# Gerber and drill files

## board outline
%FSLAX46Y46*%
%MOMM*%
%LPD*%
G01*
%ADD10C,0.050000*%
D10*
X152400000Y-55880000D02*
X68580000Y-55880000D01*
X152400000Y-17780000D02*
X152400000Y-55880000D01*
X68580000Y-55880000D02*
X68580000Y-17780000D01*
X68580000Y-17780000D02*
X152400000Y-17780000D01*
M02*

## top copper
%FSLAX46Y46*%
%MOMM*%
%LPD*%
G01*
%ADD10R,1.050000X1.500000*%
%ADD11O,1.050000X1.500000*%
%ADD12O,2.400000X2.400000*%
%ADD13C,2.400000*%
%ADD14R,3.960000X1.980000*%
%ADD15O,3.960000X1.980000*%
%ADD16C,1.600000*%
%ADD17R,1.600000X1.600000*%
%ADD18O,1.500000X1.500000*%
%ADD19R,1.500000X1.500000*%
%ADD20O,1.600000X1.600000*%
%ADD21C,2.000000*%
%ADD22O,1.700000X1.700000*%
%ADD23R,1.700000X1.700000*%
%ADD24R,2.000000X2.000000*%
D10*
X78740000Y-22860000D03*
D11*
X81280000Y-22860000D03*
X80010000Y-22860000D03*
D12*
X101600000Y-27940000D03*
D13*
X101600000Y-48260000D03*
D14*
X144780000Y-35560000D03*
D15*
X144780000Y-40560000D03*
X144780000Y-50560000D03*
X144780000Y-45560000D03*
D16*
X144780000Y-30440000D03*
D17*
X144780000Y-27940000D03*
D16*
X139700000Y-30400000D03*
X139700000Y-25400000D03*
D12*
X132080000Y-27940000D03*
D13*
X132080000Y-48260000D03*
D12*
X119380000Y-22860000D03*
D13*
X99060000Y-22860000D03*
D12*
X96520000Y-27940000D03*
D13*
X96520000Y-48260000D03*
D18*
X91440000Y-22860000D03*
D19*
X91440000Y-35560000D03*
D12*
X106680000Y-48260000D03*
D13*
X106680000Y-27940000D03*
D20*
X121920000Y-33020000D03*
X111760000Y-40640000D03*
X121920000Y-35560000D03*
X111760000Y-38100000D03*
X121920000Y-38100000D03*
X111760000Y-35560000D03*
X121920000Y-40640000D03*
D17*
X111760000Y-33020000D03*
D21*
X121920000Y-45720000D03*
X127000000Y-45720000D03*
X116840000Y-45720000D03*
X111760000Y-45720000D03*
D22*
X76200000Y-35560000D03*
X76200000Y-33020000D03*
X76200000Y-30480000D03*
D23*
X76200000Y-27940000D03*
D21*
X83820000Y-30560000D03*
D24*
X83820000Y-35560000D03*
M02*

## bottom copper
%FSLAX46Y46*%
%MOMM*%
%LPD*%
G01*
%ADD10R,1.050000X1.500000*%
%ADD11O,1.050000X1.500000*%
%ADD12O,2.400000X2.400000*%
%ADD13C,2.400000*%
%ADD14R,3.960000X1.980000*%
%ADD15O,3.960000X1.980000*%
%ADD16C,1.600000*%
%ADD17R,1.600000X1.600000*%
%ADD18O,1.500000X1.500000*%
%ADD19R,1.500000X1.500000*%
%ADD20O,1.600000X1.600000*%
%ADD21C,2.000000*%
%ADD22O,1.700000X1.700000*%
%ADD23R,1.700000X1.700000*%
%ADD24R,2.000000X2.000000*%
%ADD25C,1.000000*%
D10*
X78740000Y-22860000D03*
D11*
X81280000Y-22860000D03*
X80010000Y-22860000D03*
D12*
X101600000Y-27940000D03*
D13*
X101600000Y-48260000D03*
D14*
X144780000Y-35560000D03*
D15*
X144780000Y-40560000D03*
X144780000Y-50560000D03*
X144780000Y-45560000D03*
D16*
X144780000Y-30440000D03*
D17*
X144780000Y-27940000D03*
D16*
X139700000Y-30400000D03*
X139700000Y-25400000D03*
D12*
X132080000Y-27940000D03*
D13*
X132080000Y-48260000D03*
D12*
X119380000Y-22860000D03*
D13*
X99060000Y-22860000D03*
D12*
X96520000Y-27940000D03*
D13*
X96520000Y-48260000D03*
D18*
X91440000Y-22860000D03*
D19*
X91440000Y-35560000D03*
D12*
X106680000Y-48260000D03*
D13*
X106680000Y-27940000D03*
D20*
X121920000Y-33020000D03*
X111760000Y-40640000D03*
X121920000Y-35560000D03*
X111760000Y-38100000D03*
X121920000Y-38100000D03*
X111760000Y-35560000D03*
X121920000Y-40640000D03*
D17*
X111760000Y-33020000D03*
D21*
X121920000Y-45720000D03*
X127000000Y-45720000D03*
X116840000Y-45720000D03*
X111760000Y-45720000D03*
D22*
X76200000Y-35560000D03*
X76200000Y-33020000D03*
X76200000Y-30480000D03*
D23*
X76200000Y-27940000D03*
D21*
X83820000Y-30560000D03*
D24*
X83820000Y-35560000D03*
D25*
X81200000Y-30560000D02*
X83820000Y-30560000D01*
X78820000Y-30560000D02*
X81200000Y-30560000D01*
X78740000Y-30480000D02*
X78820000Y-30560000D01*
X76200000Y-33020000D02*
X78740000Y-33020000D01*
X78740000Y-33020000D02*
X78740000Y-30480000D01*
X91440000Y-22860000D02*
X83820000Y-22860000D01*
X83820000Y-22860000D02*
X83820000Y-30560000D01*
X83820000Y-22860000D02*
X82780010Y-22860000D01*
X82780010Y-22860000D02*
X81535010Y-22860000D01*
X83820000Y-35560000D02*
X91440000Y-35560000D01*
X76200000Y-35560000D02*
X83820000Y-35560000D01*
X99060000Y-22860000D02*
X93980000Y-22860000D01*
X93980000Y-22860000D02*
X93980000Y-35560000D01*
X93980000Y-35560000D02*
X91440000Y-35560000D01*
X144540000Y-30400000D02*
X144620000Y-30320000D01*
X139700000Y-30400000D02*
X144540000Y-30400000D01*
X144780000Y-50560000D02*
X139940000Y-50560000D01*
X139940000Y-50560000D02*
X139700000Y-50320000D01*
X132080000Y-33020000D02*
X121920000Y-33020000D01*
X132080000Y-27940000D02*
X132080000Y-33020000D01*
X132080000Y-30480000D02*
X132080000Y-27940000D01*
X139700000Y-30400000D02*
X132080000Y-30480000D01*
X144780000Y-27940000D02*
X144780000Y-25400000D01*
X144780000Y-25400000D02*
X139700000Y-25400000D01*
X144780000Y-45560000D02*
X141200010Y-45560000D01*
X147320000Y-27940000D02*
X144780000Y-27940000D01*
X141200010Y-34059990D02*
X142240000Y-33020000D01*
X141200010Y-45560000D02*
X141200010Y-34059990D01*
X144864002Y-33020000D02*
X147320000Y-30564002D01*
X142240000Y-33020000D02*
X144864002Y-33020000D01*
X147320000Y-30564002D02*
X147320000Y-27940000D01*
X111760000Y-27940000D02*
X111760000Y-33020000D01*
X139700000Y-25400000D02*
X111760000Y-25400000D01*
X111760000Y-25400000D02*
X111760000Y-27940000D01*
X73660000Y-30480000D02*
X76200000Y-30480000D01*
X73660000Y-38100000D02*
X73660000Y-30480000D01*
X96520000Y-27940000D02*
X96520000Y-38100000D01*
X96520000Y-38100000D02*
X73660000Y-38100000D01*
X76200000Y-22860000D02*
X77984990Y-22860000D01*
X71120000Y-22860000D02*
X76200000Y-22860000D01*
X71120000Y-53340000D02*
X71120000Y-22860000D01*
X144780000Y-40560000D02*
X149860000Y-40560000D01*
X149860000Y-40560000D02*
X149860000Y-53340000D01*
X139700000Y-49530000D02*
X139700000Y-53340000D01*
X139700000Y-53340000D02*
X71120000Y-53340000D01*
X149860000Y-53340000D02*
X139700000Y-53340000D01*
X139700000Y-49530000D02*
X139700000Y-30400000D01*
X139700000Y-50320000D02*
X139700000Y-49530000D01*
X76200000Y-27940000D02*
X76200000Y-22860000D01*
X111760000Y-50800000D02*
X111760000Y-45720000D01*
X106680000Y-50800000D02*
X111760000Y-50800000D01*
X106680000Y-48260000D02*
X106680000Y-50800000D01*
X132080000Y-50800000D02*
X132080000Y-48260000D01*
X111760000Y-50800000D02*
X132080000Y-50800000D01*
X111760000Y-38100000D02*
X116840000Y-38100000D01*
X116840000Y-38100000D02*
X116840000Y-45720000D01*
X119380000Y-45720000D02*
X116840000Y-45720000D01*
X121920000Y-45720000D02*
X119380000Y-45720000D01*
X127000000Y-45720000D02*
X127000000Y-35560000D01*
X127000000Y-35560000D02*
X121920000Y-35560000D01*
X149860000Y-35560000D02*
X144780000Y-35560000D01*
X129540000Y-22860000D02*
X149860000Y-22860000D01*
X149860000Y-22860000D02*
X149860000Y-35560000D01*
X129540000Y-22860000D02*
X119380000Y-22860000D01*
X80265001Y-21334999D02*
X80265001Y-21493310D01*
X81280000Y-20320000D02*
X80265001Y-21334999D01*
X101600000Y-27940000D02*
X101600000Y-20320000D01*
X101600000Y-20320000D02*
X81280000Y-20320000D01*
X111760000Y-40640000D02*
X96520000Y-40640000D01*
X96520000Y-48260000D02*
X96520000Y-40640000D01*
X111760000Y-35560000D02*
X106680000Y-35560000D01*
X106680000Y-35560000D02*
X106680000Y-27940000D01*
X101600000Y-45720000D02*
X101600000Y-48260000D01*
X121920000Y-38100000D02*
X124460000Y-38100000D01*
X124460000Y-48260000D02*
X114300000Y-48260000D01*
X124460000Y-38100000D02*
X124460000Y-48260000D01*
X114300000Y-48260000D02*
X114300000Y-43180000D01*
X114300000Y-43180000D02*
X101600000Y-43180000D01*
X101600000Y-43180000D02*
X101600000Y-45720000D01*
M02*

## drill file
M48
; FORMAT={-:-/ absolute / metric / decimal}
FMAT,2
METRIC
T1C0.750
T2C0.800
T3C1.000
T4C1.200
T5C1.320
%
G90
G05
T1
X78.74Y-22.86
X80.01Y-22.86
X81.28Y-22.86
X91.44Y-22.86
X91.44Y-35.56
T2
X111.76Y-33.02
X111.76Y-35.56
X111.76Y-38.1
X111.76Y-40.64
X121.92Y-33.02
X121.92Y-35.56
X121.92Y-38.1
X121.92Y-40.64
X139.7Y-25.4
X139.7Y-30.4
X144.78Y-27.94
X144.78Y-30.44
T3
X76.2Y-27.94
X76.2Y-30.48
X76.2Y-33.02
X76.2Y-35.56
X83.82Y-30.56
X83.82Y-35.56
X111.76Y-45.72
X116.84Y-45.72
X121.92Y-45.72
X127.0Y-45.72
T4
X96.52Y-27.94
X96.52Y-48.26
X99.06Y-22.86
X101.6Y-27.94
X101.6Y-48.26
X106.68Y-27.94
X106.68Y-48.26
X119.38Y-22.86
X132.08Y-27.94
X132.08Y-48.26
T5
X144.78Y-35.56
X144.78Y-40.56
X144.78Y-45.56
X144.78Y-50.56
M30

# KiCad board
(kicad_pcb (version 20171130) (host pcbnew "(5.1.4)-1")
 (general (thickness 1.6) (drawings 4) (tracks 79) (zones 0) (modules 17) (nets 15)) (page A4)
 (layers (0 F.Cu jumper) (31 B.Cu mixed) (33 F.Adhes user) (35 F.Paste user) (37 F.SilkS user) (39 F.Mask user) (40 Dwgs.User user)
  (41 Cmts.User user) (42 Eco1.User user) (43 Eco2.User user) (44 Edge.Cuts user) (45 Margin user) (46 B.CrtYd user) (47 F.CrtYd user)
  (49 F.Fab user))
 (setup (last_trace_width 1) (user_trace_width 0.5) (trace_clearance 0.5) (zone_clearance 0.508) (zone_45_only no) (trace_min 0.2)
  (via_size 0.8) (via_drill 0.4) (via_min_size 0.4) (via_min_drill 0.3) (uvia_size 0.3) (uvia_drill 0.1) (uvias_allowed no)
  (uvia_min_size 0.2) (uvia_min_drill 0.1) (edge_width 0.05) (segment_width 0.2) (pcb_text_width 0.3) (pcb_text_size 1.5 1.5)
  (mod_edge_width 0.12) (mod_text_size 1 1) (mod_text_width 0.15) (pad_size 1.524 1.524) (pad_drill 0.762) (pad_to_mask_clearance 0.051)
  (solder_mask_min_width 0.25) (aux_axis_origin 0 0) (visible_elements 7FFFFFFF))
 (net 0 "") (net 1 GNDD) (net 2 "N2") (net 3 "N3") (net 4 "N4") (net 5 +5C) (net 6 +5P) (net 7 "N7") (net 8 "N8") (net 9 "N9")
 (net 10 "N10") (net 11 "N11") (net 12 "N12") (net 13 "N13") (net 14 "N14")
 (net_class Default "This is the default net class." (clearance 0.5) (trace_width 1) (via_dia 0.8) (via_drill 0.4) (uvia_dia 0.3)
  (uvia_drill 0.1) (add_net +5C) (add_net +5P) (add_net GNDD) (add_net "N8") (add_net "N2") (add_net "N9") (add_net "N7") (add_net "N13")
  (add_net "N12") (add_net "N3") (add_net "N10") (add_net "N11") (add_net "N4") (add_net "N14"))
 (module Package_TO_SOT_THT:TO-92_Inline (layer F.Cu) (at 78.74 22.86)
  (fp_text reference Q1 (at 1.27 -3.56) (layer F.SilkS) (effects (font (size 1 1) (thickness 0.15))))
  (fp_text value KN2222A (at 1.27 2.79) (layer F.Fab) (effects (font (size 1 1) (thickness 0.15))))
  (pad 1 thru_hole rect (at 0 0) (size 1.05 1.5) (drill 0.75) (layers *.Cu *.Mask) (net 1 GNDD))
  (pad 3 thru_hole oval (at 2.54 0) (size 1.05 1.5) (drill 0.75) (layers *.Cu *.Mask) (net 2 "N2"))
  (pad 2 thru_hole oval (at 1.27 0) (size 1.05 1.5) (drill 0.75) (layers *.Cu *.Mask) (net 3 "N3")))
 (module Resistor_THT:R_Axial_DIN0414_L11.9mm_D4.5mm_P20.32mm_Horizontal (layer F.Cu) (at 101.6 48.26 90)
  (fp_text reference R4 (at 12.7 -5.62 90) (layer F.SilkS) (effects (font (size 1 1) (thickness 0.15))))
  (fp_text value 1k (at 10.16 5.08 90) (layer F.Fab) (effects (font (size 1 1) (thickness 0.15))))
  (pad 2 thru_hole oval (at 20.32 0 90) (size 2.4 2.4) (drill 1.2) (layers *.Cu *.Mask) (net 3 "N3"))
  (pad 1 thru_hole circle (at 0 0 90) (size 2.4 2.4) (drill 1.2) (layers *.Cu *.Mask) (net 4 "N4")))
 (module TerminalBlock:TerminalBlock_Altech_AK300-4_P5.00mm (layer F.Cu) (at 144.78 35.56 270)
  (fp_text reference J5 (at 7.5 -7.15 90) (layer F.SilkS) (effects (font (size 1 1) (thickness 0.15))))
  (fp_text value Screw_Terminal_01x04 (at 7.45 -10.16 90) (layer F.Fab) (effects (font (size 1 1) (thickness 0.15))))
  (pad 1 thru_hole rect (at 0 0 270) (size 1.98 3.96) (drill 1.32) (layers *.Cu *.Mask) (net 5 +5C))
  (pad 2 thru_hole oval (at 5 0 270) (size 1.98 3.96) (drill 1.32) (layers *.Cu *.Mask) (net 1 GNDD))
  (pad 4 thru_hole oval (at 15 0 270) (size 1.98 3.96) (drill 1.32) (layers *.Cu *.Mask) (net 1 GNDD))
  (pad 3 thru_hole oval (at 10 0 270) (size 1.98 3.96) (drill 1.32) (layers *.Cu *.Mask) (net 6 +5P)))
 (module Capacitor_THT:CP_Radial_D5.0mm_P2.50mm (layer F.Cu) (at 144.78 27.94 270)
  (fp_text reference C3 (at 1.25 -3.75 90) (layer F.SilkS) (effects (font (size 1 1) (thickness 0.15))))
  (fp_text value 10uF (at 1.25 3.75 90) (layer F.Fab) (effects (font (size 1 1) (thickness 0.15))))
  (pad 2 thru_hole circle (at 2.5 0 270) (size 1.6 1.6) (drill 0.8) (layers *.Cu *.Mask) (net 1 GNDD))
  (pad 1 thru_hole rect (at 0 0 270) (size 1.6 1.6) (drill 0.8) (layers *.Cu *.Mask) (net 6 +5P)))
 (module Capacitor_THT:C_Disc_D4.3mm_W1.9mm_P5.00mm (layer F.Cu) (at 139.7 25.4 270)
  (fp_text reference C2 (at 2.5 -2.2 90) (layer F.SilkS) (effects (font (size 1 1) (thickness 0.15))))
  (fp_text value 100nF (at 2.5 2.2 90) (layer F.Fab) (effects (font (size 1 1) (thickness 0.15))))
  (pad 2 thru_hole circle (at 5 0 270) (size 1.6 1.6) (drill 0.8) (layers *.Cu *.Mask) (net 1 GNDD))
  (pad 1 thru_hole circle (at 0 0 270) (size 1.6 1.6) (drill 0.8) (layers *.Cu *.Mask) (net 6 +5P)))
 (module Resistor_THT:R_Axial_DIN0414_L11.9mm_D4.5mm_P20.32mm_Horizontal (layer F.Cu) (at 132.08 48.26 90)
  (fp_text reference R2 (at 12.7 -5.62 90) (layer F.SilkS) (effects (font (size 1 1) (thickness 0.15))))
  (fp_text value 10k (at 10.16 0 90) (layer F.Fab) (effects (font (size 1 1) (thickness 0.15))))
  (pad 2 thru_hole oval (at 20.32 0 90) (size 2.4 2.4) (drill 1.2) (layers *.Cu *.Mask) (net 1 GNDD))
  (pad 1 thru_hole circle (at 0 0 90) (size 2.4 2.4) (drill 1.2) (layers *.Cu *.Mask) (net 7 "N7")))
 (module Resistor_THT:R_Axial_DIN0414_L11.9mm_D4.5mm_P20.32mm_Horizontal (layer F.Cu) (at 99.06 22.86)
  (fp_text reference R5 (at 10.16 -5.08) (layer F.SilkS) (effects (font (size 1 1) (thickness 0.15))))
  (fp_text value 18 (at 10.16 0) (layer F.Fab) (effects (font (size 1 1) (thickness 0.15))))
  (pad 2 thru_hole oval (at 20.32 0) (size 2.4 2.4) (drill 1.2) (layers *.Cu *.Mask) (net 5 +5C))
  (pad 1 thru_hole circle (at 0 0) (size 2.4 2.4) (drill 1.2) (layers *.Cu *.Mask) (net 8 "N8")))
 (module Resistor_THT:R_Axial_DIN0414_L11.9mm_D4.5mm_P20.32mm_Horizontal (layer F.Cu) (at 96.52 48.26 90)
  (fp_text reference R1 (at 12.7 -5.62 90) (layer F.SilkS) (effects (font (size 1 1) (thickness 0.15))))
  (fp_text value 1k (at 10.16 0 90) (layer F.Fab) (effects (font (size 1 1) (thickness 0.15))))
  (pad 2 thru_hole oval (at 20.32 0 90) (size 2.4 2.4) (drill 1.2) (layers *.Cu *.Mask) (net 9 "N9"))
  (pad 1 thru_hole circle (at 0 0 90) (size 2.4 2.4) (drill 1.2) (layers *.Cu *.Mask) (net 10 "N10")))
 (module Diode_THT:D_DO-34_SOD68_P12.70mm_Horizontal (layer F.Cu) (at 91.44 35.56 90)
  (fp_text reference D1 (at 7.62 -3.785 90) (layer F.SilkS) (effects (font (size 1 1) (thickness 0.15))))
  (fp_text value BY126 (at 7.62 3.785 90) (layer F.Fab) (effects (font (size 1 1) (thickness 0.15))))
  (pad 2 thru_hole oval (at 12.7 0 90) (size 1.5 1.5) (drill 0.75) (layers *.Cu *.Mask) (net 2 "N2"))
  (pad 1 thru_hole rect (at 0 0 90) (size 1.5 1.5) (drill 0.75) (layers *.Cu *.Mask) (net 8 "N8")))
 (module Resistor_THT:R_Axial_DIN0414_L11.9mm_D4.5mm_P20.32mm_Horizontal (layer F.Cu) (at 106.68 27.94 270)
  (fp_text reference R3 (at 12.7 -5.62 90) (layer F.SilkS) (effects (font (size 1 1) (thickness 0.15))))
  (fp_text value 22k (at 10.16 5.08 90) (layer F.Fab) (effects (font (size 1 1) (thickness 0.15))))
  (pad 2 thru_hole oval (at 20.32 0 270) (size 2.4 2.4) (drill 1.2) (layers *.Cu *.Mask) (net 7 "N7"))
  (pad 1 thru_hole circle (at 0 0 270) (size 2.4 2.4) (drill 1.2) (layers *.Cu *.Mask) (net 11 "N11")))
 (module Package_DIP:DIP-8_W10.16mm (layer F.Cu) (at 111.76 33.02)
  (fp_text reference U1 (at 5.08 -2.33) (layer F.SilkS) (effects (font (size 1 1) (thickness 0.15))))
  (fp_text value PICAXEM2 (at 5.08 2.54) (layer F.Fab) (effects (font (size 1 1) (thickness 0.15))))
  (pad 8 thru_hole oval (at 10.16 0) (size 1.6 1.6) (drill 0.8) (layers *.Cu *.Mask) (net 1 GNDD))
  (pad 4 thru_hole oval (at 0 7.62) (size 1.6 1.6) (drill 0.8) (layers *.Cu *.Mask) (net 10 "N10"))
  (pad 7 thru_hole oval (at 10.16 2.54) (size 1.6 1.6) (drill 0.8) (layers *.Cu *.Mask) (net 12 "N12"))
  (pad 3 thru_hole oval (at 0 5.08) (size 1.6 1.6) (drill 0.8) (layers *.Cu *.Mask) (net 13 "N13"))
  (pad 6 thru_hole oval (at 10.16 5.08) (size 1.6 1.6) (drill 0.8) (layers *.Cu *.Mask) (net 4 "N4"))
  (pad 2 thru_hole oval (at 0 2.54) (size 1.6 1.6) (drill 0.8) (layers *.Cu *.Mask) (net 11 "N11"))
  (pad 5 thru_hole oval (at 10.16 7.62) (size 1.6 1.6) (drill 0.8) (layers *.Cu *.Mask) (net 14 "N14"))
  (pad 1 thru_hole rect (at 0 0) (size 1.6 1.6) (drill 0.8) (layers *.Cu *.Mask) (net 6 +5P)))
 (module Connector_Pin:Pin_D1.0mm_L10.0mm (layer F.Cu) (at 121.92 45.72)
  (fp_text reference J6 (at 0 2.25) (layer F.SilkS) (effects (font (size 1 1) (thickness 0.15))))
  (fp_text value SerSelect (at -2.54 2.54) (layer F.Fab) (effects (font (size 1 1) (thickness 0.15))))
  (pad 1 thru_hole circle (at 0 0) (size 2 2) (drill 1) (layers *.Cu *.Mask) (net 13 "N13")))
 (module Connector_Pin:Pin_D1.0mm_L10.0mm (layer F.Cu) (at 127 45.72)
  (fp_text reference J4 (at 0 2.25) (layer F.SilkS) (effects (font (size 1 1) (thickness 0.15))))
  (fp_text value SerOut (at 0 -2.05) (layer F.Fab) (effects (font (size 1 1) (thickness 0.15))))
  (pad 1 thru_hole circle (at 0 0) (size 2 2) (drill 1) (layers *.Cu *.Mask) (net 12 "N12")))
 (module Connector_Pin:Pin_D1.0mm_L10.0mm (layer F.Cu) (at 116.84 45.72)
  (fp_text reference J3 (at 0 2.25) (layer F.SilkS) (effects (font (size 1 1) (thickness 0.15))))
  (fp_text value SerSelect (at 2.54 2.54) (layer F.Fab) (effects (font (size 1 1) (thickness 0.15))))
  (pad 1 thru_hole circle (at 0 0) (size 2 2) (drill 1) (layers *.Cu *.Mask) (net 13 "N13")))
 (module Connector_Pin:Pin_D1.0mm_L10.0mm (layer F.Cu) (at 111.76 45.72)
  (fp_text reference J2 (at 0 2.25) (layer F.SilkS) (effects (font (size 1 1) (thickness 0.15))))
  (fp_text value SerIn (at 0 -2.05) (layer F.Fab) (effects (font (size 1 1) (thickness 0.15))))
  (pad 1 thru_hole circle (at 0 0) (size 2 2) (drill 1) (layers *.Cu *.Mask) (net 7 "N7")))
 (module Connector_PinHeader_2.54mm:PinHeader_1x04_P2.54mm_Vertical (layer F.Cu) (at 76.2 27.94)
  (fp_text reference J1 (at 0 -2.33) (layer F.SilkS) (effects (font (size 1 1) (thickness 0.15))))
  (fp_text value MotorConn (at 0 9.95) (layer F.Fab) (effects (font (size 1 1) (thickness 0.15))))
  (pad 4 thru_hole oval (at 0 7.62) (size 1.7 1.7) (drill 1) (layers *.Cu *.Mask) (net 8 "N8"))
  (pad 3 thru_hole oval (at 0 5.08) (size 1.7 1.7) (drill 1) (layers *.Cu *.Mask) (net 2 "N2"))
  (pad 2 thru_hole oval (at 0 2.54) (size 1.7 1.7) (drill 1) (layers *.Cu *.Mask) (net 9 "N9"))
  (pad 1 thru_hole rect (at 0 0) (size 1.7 1.7) (drill 1) (layers *.Cu *.Mask) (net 1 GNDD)))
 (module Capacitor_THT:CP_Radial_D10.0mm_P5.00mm (layer F.Cu) (at 83.82 35.56 90)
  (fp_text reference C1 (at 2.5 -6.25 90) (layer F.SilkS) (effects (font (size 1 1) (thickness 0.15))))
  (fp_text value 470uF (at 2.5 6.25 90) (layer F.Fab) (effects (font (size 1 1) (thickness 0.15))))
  (pad 2 thru_hole circle (at 5 0 90) (size 2 2) (drill 1) (layers *.Cu *.Mask) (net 2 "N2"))
  (pad 1 thru_hole rect (at 0 0 90) (size 2 2) (drill 1) (layers *.Cu *.Mask) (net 8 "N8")))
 (gr_line (start 152.4 55.88) (end 68.58 55.88) (layer Edge.Cuts) (width 0.05))
 (gr_line (start 152.4 17.78) (end 152.4 55.88) (layer Edge.Cuts) (width 0.05))
 (gr_line (start 68.58 55.88) (end 68.58 17.78) (layer Edge.Cuts) (width 0.05))
 (gr_line (start 68.58 17.78) (end 152.4 17.78) (layer Edge.Cuts) (width 0.05))
 (segment (start 81.2 30.56) (end 83.82 30.56) (width 1) (layer B.Cu) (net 2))
 (segment (start 78.82 30.56) (end 81.2 30.56) (width 1) (layer B.Cu) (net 2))
 (segment (start 78.74 30.48) (end 78.82 30.56) (width 1) (layer B.Cu) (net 2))
 (segment (start 76.2 33.02) (end 78.74 33.02) (width 1) (layer B.Cu) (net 2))
 (segment (start 78.74 33.02) (end 78.74 30.48) (width 1) (layer B.Cu) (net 2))
 (segment (start 91.44 22.86) (end 83.82 22.86) (width 1) (layer B.Cu) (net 2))
 (segment (start 83.82 22.86) (end 83.82 30.56) (width 1) (layer B.Cu) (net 2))
 (segment (start 83.82 22.86) (end 82.78001 22.86) (width 1) (layer B.Cu) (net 2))
 (segment (start 82.78001 22.86) (end 81.53501 22.86) (width 1) (layer B.Cu) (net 2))
 (segment (start 83.82 35.56) (end 91.44 35.56) (width 1) (layer B.Cu) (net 8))
 (segment (start 76.2 35.56) (end 83.82 35.56) (width 1) (layer B.Cu) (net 8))
 (segment (start 99.06 22.86) (end 93.98 22.86) (width 1) (layer B.Cu) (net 8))
 (segment (start 93.98 22.86) (end 93.98 35.56) (width 1) (layer B.Cu) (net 8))
 (segment (start 93.98 35.56) (end 91.44 35.56) (width 1) (layer B.Cu) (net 8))
 (segment (start 144.54 30.4) (end 144.62 30.32) (width 1) (layer B.Cu) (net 1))
 (segment (start 139.7 30.4) (end 144.54 30.4) (width 1) (layer B.Cu) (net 1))
 (segment (start 144.78 50.56) (end 139.94 50.56) (width 1) (layer B.Cu) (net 1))
 (segment (start 139.94 50.56) (end 139.7 50.32) (width 1) (layer B.Cu) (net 1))
 (segment (start 132.08 33.02) (end 121.92 33.02) (width 1) (layer B.Cu) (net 1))
 (segment (start 132.08 27.94) (end 132.08 33.02) (width 1) (layer B.Cu) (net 1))
 (segment (start 132.08 30.48) (end 132.08 27.94) (width 1) (layer B.Cu) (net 1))
 (segment (start 139.7 30.4) (end 132.08 30.48) (width 1) (layer B.Cu) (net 1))
 (segment (start 144.78 27.94) (end 144.78 25.4) (width 1) (layer B.Cu) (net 6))
 (segment (start 144.78 25.4) (end 139.7 25.4) (width 1) (layer B.Cu) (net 6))
 (segment (start 144.78 45.56) (end 141.20001 45.56) (width 1) (layer B.Cu) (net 6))
 (segment (start 147.32 27.94) (end 144.78 27.94) (width 1) (layer B.Cu) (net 6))
 (segment (start 141.20001 34.05999) (end 142.24 33.02) (width 1) (layer B.Cu) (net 6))
 (segment (start 141.20001 45.56) (end 141.20001 34.05999) (width 1) (layer B.Cu) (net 6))
 (segment (start 144.864002 33.02) (end 147.32 30.564002) (width 1) (layer B.Cu) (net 6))
 (segment (start 142.24 33.02) (end 144.864002 33.02) (width 1) (layer B.Cu) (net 6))
 (segment (start 147.32 30.564002) (end 147.32 27.94) (width 1) (layer B.Cu) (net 6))
 (segment (start 111.76 27.94) (end 111.76 33.02) (width 1) (layer B.Cu) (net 6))
 (segment (start 139.7 25.4) (end 111.76 25.4) (width 1) (layer B.Cu) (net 6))
 (segment (start 111.76 25.4) (end 111.76 27.94) (width 1) (layer B.Cu) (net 6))
 (segment (start 73.66 30.48) (end 76.2 30.48) (width 1) (layer B.Cu) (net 9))
 (segment (start 73.66 38.1) (end 73.66 30.48) (width 1) (layer B.Cu) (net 9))
 (segment (start 96.52 27.94) (end 96.52 38.1) (width 1) (layer B.Cu) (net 9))
 (segment (start 96.52 38.1) (end 73.66 38.1) (width 1) (layer B.Cu) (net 9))
 (segment (start 76.2 22.86) (end 77.98499 22.86) (width 1) (layer B.Cu) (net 1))
 (segment (start 71.12 22.86) (end 76.2 22.86) (width 1) (layer B.Cu) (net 1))
 (segment (start 71.12 53.34) (end 71.12 22.86) (width 1) (layer B.Cu) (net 1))
 (segment (start 144.78 40.56) (end 149.86 40.56) (width 1) (layer B.Cu) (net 1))
 (segment (start 149.86 40.56) (end 149.86 53.34) (width 1) (layer B.Cu) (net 1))
 (segment (start 139.7 49.53) (end 139.7 53.34) (width 1) (layer B.Cu) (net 1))
 (segment (start 139.7 53.34) (end 71.12 53.34) (width 1) (layer B.Cu) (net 1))
 (segment (start 149.86 53.34) (end 139.7 53.34) (width 1) (layer B.Cu) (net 1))
 (segment (start 139.7 49.53) (end 139.7 30.4) (width 1) (layer B.Cu) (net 1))
 (segment (start 139.7 50.32) (end 139.7 49.53) (width 1) (layer B.Cu) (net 1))
 (segment (start 76.2 27.94) (end 76.2 22.86) (width 1) (layer B.Cu) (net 1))
 (segment (start 111.76 50.8) (end 111.76 45.72) (width 1) (layer B.Cu) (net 7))
 (segment (start 106.68 50.8) (end 111.76 50.8) (width 1) (layer B.Cu) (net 7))
 (segment (start 106.68 48.26) (end 106.68 50.8) (width 1) (layer B.Cu) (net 7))
 (segment (start 132.08 50.8) (end 132.08 48.26) (width 1) (layer B.Cu) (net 7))
 (segment (start 111.76 50.8) (end 132.08 50.8) (width 1) (layer B.Cu) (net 7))
 (segment (start 111.76 38.1) (end 116.84 38.1) (width 1) (layer B.Cu) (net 13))
 (segment (start 116.84 38.1) (end 116.84 45.72) (width 1) (layer B.Cu) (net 13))
 (segment (start 119.38 45.72) (end 116.84 45.72) (width 1) (layer B.Cu) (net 13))
 (segment (start 121.92 45.72) (end 119.38 45.72) (width 1) (layer B.Cu) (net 13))
 (segment (start 127 45.72) (end 127 35.56) (width 1) (layer B.Cu) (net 12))
 (segment (start 127 35.56) (end 121.92 35.56) (width 1) (layer B.Cu) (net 12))
 (segment (start 149.86 35.56) (end 144.78 35.56) (width 1) (layer B.Cu) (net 5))
 (segment (start 129.54 22.86) (end 149.86 22.86) (width 1) (layer B.Cu) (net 5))
 (segment (start 149.86 22.86) (end 149.86 35.56) (width 1) (layer B.Cu) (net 5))
 (segment (start 129.54 22.86) (end 119.38 22.86) (width 1) (layer B.Cu) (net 5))
 (segment (start 80.265001 21.334999) (end 80.265001 21.49331) (width 1) (layer B.Cu) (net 3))
 (segment (start 81.28 20.32) (end 80.265001 21.334999) (width 1) (layer B.Cu) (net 3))
 (segment (start 101.6 27.94) (end 101.6 20.32) (width 1) (layer B.Cu) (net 3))
 (segment (start 101.6 20.32) (end 81.28 20.32) (width 1) (layer B.Cu) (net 3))
 (segment (start 111.76 40.64) (end 96.52 40.64) (width 1) (layer B.Cu) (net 10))
 (segment (start 96.52 48.26) (end 96.52 40.64) (width 1) (layer B.Cu) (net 10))
 (segment (start 111.76 35.56) (end 106.68 35.56) (width 1) (layer B.Cu) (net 11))
 (segment (start 106.68 35.56) (end 106.68 27.94) (width 1) (layer B.Cu) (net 11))
 (segment (start 101.6 45.72) (end 101.6 48.26) (width 1) (layer B.Cu) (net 4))
 (segment (start 121.92 38.1) (end 124.46 38.1) (width 1) (layer B.Cu) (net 4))
 (segment (start 124.46 48.26) (end 114.3 48.26) (width 1) (layer B.Cu) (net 4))
 (segment (start 124.46 38.1) (end 124.46 48.26) (width 1) (layer B.Cu) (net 4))
 (segment (start 114.3 48.26) (end 114.3 43.18) (width 1) (layer B.Cu) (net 4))
 (segment (start 114.3 43.18) (end 101.6 43.18) (width 1) (layer B.Cu) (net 4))
 (segment (start 101.6 43.18) (end 101.6 45.72) (width 1) (layer B.Cu) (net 4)))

